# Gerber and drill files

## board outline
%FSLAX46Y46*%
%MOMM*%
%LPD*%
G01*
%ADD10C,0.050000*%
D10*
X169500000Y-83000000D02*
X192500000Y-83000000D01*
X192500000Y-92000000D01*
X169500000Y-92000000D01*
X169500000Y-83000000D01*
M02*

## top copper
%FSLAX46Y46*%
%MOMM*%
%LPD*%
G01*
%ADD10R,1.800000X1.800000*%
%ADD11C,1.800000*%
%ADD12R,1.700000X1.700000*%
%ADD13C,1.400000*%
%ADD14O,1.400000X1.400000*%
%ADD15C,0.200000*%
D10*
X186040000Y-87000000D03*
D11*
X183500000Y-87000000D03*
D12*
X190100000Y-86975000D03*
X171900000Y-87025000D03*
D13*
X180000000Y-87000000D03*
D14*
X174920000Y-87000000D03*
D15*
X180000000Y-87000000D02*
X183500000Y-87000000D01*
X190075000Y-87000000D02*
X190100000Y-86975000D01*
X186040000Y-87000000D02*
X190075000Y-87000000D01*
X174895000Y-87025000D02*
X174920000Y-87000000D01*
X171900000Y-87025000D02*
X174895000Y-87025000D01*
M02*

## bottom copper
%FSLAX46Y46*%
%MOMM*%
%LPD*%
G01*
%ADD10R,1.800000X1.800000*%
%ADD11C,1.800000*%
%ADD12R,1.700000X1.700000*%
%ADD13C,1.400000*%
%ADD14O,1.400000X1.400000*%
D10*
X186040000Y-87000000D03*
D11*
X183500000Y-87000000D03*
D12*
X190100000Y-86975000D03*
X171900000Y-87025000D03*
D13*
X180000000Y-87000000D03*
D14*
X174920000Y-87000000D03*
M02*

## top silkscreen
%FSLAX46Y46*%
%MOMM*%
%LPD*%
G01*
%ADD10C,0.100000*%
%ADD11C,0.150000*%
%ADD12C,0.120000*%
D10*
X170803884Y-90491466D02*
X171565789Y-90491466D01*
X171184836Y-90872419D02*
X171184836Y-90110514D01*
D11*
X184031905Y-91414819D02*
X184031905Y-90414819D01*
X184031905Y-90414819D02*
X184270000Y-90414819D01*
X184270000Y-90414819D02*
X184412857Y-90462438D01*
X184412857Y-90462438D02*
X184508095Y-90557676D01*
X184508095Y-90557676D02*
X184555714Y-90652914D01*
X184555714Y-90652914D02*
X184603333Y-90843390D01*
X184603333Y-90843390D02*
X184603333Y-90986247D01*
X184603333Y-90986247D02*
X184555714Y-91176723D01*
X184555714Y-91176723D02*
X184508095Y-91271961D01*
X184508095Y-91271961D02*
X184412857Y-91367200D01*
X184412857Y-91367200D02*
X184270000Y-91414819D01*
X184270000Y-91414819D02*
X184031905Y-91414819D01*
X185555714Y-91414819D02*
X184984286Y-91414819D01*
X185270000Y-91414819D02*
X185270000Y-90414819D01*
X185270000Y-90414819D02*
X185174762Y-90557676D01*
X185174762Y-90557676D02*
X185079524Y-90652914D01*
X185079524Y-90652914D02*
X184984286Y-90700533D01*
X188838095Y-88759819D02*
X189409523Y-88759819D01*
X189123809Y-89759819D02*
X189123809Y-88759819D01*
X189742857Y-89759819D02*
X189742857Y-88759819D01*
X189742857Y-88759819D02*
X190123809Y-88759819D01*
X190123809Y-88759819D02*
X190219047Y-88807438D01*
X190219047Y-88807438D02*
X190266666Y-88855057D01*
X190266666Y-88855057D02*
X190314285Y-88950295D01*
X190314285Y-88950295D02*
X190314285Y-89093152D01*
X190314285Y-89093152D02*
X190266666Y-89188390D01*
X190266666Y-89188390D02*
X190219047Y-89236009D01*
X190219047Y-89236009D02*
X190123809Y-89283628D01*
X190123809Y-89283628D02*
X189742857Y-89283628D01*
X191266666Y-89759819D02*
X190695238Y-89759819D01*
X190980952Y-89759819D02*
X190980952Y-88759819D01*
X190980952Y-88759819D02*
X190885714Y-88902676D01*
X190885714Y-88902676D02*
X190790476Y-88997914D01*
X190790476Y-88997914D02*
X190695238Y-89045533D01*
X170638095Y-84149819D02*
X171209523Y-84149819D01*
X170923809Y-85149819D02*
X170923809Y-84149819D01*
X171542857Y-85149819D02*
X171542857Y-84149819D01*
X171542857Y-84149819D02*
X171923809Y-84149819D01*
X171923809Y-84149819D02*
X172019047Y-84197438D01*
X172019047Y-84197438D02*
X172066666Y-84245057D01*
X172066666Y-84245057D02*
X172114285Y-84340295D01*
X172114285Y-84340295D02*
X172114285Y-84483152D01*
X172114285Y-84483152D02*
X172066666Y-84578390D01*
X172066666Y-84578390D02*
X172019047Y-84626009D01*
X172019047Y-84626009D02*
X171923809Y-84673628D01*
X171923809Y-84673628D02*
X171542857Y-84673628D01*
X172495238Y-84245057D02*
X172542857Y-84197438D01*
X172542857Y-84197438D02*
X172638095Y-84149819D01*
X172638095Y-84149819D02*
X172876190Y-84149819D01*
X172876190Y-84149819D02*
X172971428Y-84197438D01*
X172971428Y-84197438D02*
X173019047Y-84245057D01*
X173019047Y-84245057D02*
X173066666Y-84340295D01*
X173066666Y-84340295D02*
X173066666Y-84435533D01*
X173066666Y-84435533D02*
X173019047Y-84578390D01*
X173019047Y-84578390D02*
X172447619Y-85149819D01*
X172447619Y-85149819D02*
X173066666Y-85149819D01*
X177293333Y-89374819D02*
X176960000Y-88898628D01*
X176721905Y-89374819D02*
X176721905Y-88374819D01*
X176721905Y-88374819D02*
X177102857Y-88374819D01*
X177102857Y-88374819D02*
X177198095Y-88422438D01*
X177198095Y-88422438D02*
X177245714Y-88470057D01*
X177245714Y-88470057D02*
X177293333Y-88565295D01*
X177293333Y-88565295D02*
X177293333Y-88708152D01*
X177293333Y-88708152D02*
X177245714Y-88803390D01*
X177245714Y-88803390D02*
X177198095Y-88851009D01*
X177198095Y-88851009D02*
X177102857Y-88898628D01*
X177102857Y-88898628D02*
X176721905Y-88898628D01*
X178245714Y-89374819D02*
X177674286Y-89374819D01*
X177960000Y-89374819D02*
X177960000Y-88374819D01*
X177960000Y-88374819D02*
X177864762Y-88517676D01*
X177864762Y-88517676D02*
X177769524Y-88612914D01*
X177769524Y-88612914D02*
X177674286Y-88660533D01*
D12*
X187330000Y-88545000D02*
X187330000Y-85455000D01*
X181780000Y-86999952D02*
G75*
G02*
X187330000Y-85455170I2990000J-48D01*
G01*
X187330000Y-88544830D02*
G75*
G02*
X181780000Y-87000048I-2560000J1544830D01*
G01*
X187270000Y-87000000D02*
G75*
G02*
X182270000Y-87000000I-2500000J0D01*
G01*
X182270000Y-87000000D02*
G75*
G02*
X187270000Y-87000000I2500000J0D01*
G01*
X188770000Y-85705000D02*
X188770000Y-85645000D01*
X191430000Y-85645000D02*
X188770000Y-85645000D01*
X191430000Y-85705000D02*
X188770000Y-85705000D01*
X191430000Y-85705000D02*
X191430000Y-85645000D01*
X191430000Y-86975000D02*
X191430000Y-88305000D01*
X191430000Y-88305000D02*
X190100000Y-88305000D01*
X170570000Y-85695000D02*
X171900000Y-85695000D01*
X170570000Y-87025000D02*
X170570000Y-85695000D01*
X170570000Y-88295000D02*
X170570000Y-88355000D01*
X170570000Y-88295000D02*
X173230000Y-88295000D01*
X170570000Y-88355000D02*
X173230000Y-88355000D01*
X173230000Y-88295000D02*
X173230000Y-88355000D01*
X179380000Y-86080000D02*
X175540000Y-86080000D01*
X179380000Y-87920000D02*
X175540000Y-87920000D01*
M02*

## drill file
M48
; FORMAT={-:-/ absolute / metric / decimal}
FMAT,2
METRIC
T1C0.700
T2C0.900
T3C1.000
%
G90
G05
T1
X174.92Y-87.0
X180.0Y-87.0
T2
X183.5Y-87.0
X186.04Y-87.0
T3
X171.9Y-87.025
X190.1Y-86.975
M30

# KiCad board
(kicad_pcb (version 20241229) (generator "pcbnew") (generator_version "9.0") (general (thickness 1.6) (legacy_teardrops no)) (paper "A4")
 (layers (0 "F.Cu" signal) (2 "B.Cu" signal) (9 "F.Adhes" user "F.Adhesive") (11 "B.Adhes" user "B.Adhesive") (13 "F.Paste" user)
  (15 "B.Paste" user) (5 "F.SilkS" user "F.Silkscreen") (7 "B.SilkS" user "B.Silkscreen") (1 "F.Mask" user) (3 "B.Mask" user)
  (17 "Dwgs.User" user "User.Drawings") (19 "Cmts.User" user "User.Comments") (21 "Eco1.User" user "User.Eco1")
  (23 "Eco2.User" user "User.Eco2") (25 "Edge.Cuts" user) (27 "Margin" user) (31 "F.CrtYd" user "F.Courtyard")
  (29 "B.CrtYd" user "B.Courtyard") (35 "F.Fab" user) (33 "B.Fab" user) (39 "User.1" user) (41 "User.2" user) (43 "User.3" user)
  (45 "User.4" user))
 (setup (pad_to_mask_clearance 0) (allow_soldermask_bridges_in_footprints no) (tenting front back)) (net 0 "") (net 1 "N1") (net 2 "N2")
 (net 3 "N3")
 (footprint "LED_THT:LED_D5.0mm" (layer "F.Cu") (at 186.04 87 180)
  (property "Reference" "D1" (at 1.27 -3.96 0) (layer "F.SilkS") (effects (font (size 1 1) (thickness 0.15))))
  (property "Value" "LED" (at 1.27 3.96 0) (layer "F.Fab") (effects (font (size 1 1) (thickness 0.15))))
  (fp_line (start -1.29 -1.545) (end -1.29 1.545) (stroke (width 0.12) (type solid)) (layer "F.SilkS"))
  (fp_arc (start 4.26 0.000048) (mid 2.071756 2.880501) (end -1.29 1.54483) (stroke (width 0.12) (type solid)) (layer "F.SilkS"))
  (fp_arc (start -1.29 -1.54483) (mid 2.071756 -2.880501) (end 4.26 -0.000048) (stroke (width 0.12) (type solid)) (layer "F.SilkS"))
  (fp_circle (center 1.27 0) (end 3.77 0) (stroke (width 0.12) (type solid)) (fill no) (layer "F.SilkS"))
  (pad "1" thru_hole rect (at 0 0 180) (size 1.8 1.8) (drill 0.9) (layers "*.Cu" "*.Mask") (remove_unused_layers no) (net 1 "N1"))
  (pad "2" thru_hole circle (at 2.54 0 180) (size 1.8 1.8) (drill 0.9) (layers "*.Cu" "*.Mask") (remove_unused_layers no) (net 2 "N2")))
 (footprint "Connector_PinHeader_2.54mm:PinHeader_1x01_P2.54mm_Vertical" (layer "F.Cu") (at 190.1 86.975 180)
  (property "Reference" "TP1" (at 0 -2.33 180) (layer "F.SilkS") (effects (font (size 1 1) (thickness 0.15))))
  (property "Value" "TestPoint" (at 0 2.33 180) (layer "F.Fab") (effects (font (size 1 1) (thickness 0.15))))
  (fp_line (start 1.33 1.27) (end 1.33 1.33) (stroke (width 0.12) (type solid)) (layer "F.SilkS"))
  (fp_line (start -1.33 1.33) (end 1.33 1.33) (stroke (width 0.12) (type solid)) (layer "F.SilkS"))
  (fp_line (start -1.33 1.27) (end 1.33 1.27) (stroke (width 0.12) (type solid)) (layer "F.SilkS"))
  (fp_line (start -1.33 1.27) (end -1.33 1.33) (stroke (width 0.12) (type solid)) (layer "F.SilkS"))
  (fp_line (start -1.33 0) (end -1.33 -1.33) (stroke (width 0.12) (type solid)) (layer "F.SilkS"))
  (fp_line (start -1.33 -1.33) (end 0 -1.33) (stroke (width 0.12) (type solid)) (layer "F.SilkS"))
  (pad "1" thru_hole rect (at 0 0 180) (size 1.7 1.7) (drill 1) (layers "*.Cu" "*.Mask") (remove_unused_layers no) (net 1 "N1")))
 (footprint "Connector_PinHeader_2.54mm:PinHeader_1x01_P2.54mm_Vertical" (layer "F.Cu") (at 171.9 87.025)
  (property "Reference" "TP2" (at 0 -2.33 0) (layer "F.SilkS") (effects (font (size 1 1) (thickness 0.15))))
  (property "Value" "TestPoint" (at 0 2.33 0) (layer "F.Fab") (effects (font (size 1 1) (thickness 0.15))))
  (fp_line (start -1.33 -1.33) (end 0 -1.33) (stroke (width 0.12) (type solid)) (layer "F.SilkS"))
  (fp_line (start -1.33 0) (end -1.33 -1.33) (stroke (width 0.12) (type solid)) (layer "F.SilkS"))
  (fp_line (start -1.33 1.27) (end -1.33 1.33) (stroke (width 0.12) (type solid)) (layer "F.SilkS"))
  (fp_line (start -1.33 1.27) (end 1.33 1.27) (stroke (width 0.12) (type solid)) (layer "F.SilkS"))
  (fp_line (start -1.33 1.33) (end 1.33 1.33) (stroke (width 0.12) (type solid)) (layer "F.SilkS"))
  (fp_line (start 1.33 1.27) (end 1.33 1.33) (stroke (width 0.12) (type solid)) (layer "F.SilkS"))
  (pad "1" thru_hole rect (at 0 0) (size 1.7 1.7) (drill 1) (layers "*.Cu" "*.Mask") (remove_unused_layers no) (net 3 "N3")))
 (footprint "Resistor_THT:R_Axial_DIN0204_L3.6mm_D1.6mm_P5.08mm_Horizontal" (layer "F.Cu") (at 180 87 180)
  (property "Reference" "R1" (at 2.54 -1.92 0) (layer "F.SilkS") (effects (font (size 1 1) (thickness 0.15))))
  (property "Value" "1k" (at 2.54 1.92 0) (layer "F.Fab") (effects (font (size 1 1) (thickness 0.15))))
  (fp_line (start 0.62 0.92) (end 4.46 0.92) (stroke (width 0.12) (type solid)) (layer "F.SilkS"))
  (fp_line (start 0.62 -0.92) (end 4.46 -0.92) (stroke (width 0.12) (type solid)) (layer "F.SilkS"))
  (pad "1" thru_hole circle (at 0 0 180) (size 1.4 1.4) (drill 0.7) (layers "*.Cu" "*.Mask") (remove_unused_layers no) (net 2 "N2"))
  (pad "2" thru_hole oval (at 5.08 0 180) (size 1.4 1.4) (drill 0.7) (layers "*.Cu" "*.Mask") (remove_unused_layers no) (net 3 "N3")))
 (gr_rect (start 169.5 83) (end 192.5 92) (stroke (width 0.05) (type default)) (fill no) (layer "Edge.Cuts"))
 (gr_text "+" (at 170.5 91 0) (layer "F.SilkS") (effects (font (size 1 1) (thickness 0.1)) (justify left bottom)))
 (segment (start 180 87) (end 183.5 87) (width 0.2) (layer "F.Cu") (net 2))
 (segment (start 190.075 87) (end 190.1 86.975) (width 0.2) (layer "F.Cu") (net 1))
 (segment (start 186.04 87) (end 190.075 87) (width 0.2) (layer "F.Cu") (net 1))
 (segment (start 174.895 87.025) (end 174.92 87) (width 0.2) (layer "F.Cu") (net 3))
 (segment (start 171.9 87.025) (end 174.895 87.025) (width 0.2) (layer "F.Cu") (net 3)))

